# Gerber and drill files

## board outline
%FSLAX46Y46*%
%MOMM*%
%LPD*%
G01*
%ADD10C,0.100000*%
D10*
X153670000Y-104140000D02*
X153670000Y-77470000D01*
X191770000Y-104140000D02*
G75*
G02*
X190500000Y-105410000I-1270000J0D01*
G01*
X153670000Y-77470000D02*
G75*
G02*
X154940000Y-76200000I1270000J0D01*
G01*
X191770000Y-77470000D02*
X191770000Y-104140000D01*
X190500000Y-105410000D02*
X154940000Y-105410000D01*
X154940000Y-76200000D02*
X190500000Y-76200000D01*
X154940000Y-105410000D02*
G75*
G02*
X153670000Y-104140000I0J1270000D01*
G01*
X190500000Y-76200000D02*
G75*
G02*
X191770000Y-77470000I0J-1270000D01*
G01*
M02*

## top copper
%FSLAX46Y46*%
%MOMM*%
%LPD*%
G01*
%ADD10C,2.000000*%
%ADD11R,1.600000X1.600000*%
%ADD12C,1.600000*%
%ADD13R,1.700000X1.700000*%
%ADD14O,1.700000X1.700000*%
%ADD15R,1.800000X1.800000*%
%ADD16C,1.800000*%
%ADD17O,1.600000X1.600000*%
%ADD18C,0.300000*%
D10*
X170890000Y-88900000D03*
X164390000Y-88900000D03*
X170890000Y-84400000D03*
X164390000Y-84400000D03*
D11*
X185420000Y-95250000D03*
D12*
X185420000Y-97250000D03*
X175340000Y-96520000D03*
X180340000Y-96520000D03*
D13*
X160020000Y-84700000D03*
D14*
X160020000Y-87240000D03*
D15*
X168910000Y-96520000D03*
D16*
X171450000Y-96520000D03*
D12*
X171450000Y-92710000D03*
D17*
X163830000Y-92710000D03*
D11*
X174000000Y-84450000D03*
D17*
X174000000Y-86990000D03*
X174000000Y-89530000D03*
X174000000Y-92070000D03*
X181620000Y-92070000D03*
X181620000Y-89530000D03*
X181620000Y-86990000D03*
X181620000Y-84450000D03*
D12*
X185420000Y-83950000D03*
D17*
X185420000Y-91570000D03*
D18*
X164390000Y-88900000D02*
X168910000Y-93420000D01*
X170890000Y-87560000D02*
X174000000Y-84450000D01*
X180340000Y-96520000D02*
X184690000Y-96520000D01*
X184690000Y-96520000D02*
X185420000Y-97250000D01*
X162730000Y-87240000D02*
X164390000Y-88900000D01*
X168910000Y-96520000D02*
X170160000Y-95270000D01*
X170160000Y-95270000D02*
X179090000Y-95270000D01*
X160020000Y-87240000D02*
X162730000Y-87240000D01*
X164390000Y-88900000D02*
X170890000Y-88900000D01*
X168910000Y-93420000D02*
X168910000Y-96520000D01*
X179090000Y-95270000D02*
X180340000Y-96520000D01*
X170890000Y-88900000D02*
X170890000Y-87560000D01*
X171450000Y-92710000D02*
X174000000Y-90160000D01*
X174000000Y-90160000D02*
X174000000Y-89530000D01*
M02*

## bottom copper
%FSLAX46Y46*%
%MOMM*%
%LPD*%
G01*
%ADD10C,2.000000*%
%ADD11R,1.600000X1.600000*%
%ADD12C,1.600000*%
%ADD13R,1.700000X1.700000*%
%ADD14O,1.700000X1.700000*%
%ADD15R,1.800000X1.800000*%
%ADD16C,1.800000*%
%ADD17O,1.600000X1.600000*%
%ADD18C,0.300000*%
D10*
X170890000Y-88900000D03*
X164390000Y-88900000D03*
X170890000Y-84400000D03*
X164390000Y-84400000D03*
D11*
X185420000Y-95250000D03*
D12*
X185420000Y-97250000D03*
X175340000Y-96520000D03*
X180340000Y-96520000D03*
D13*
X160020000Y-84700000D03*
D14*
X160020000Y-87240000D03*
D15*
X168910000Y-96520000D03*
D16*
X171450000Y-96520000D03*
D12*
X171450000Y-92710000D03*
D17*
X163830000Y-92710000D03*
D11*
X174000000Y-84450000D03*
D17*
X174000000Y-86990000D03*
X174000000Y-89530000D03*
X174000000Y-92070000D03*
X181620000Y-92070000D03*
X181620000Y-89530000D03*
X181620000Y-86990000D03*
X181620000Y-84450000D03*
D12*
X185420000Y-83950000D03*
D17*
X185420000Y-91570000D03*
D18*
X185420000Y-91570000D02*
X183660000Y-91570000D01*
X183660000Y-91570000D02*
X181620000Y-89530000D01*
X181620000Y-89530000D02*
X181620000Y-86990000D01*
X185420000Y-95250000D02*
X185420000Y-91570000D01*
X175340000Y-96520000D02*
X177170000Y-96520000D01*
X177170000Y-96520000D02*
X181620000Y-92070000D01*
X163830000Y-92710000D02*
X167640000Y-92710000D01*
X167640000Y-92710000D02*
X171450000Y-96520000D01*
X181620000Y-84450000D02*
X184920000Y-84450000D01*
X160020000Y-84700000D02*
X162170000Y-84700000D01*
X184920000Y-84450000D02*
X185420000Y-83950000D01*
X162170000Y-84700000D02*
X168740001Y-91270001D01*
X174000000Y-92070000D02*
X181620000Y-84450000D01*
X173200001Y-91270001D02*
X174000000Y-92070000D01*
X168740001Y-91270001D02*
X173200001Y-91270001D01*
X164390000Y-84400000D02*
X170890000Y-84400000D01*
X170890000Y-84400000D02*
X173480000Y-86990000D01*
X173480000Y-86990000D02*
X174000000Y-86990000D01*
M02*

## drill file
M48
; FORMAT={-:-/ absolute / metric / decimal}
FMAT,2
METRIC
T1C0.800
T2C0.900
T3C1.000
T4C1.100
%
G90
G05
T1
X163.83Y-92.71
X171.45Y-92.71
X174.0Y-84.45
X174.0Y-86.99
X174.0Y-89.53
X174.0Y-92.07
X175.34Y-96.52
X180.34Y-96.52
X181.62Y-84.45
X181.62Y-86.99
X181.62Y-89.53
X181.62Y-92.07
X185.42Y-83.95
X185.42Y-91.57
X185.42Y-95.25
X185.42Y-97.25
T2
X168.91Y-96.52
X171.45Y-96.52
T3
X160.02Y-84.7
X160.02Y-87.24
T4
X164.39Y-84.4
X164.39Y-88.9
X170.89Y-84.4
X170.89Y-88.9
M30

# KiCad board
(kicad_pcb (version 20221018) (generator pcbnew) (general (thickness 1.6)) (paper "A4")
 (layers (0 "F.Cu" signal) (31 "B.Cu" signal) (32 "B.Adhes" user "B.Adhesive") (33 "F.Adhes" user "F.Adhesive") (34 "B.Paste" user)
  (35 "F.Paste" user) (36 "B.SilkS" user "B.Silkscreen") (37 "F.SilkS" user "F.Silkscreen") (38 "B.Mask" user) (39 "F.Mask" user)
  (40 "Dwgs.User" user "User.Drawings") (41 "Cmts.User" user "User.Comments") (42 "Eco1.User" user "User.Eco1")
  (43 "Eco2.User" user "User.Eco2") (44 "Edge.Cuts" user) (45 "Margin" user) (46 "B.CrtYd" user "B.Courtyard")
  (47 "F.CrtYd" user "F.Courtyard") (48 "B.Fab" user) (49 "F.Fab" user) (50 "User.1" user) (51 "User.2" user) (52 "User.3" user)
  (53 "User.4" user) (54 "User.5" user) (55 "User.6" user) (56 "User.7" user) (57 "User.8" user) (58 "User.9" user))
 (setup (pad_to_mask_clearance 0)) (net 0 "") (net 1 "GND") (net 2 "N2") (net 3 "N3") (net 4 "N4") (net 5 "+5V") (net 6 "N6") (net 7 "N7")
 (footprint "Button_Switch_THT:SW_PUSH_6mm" (layer "F.Cu") (at 170.89 88.9 180)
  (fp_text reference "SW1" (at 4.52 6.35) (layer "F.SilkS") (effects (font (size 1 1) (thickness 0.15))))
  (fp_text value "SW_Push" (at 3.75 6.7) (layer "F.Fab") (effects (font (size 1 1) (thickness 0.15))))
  (pad "1" thru_hole circle (at 0 0 270) (size 2 2) (drill 1.1) (layers "*.Cu" "*.Mask") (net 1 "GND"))
  (pad "1" thru_hole circle (at 6.5 0 270) (size 2 2) (drill 1.1) (layers "*.Cu" "*.Mask") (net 1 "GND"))
  (pad "2" thru_hole circle (at 0 4.5 270) (size 2 2) (drill 1.1) (layers "*.Cu" "*.Mask") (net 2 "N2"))
  (pad "2" thru_hole circle (at 6.5 4.5 270) (size 2 2) (drill 1.1) (layers "*.Cu" "*.Mask") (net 2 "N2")))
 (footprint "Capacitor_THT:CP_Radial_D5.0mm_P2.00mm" (layer "F.Cu") (at 185.42 95.25 -90)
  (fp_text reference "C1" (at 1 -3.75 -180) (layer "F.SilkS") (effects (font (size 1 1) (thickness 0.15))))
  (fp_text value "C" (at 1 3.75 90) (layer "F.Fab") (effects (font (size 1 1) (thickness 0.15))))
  (pad "1" thru_hole rect (at 0 0 270) (size 1.6 1.6) (drill 0.8) (layers "*.Cu" "*.Mask") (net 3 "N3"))
  (pad "2" thru_hole circle (at 2 0 270) (size 1.6 1.6) (drill 0.8) (layers "*.Cu" "*.Mask") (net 1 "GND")))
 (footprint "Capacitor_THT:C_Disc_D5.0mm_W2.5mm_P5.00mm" (layer "F.Cu") (at 175.34 96.52)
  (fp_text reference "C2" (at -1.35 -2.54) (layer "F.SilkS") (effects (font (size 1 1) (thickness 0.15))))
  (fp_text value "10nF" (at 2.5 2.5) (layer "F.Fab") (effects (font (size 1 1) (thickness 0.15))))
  (pad "1" thru_hole circle (at 0 0) (size 1.6 1.6) (drill 0.8) (layers "*.Cu" "*.Mask") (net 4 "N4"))
  (pad "2" thru_hole circle (at 5 0) (size 1.6 1.6) (drill 0.8) (layers "*.Cu" "*.Mask") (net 1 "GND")))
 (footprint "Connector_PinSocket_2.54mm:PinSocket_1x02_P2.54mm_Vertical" (layer "F.Cu") (at 160.02 84.7)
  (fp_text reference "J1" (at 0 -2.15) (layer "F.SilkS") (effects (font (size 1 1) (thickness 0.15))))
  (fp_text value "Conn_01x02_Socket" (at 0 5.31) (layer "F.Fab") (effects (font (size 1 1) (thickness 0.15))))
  (pad "1" thru_hole rect (at 0 0) (size 1.7 1.7) (drill 1) (layers "*.Cu" "*.Mask") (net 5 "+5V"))
  (pad "2" thru_hole oval (at 0 2.54) (size 1.7 1.7) (drill 1) (layers "*.Cu" "*.Mask") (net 1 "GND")))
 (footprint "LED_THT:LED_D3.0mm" (layer "F.Cu") (at 168.91 96.52)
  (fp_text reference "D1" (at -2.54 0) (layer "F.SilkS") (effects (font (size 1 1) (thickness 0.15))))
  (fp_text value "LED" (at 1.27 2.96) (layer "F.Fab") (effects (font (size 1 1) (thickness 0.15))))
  (pad "1" thru_hole rect (at 0 0) (size 1.8 1.8) (drill 0.9) (layers "*.Cu" "*.Mask") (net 1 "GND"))
  (pad "2" thru_hole circle (at 2.54 0) (size 1.8 1.8) (drill 0.9) (layers "*.Cu" "*.Mask") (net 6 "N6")))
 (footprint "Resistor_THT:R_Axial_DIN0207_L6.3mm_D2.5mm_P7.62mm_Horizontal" (layer "F.Cu") (at 171.45 92.71 180)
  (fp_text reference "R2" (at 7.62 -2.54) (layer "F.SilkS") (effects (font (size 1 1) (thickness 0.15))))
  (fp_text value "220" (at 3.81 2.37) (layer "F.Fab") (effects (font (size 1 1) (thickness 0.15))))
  (pad "1" thru_hole circle (at 0 0 180) (size 1.6 1.6) (drill 0.8) (layers "*.Cu" "*.Mask") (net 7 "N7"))
  (pad "2" thru_hole oval (at 7.62 0 180) (size 1.6 1.6) (drill 0.8) (layers "*.Cu" "*.Mask") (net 6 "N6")))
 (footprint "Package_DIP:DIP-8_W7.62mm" (layer "F.Cu") (at 174 84.45)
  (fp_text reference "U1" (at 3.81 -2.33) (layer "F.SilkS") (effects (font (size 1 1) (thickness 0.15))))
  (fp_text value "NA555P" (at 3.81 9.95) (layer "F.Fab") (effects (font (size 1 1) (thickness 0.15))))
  (pad "1" thru_hole rect (at 0 0) (size 1.6 1.6) (drill 0.8) (layers "*.Cu" "*.Mask") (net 1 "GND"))
  (pad "2" thru_hole oval (at 0 2.54) (size 1.6 1.6) (drill 0.8) (layers "*.Cu" "*.Mask") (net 2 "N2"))
  (pad "3" thru_hole oval (at 0 5.08) (size 1.6 1.6) (drill 0.8) (layers "*.Cu" "*.Mask") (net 7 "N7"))
  (pad "4" thru_hole oval (at 0 7.62) (size 1.6 1.6) (drill 0.8) (layers "*.Cu" "*.Mask") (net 5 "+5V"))
  (pad "5" thru_hole oval (at 7.62 7.62) (size 1.6 1.6) (drill 0.8) (layers "*.Cu" "*.Mask") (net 4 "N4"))
  (pad "6" thru_hole oval (at 7.62 5.08) (size 1.6 1.6) (drill 0.8) (layers "*.Cu" "*.Mask") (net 3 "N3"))
  (pad "7" thru_hole oval (at 7.62 2.54) (size 1.6 1.6) (drill 0.8) (layers "*.Cu" "*.Mask") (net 3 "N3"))
  (pad "8" thru_hole oval (at 7.62 0) (size 1.6 1.6) (drill 0.8) (layers "*.Cu" "*.Mask") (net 5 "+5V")))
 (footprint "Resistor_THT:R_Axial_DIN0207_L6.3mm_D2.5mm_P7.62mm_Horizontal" (layer "F.Cu") (at 185.42 83.95 -90)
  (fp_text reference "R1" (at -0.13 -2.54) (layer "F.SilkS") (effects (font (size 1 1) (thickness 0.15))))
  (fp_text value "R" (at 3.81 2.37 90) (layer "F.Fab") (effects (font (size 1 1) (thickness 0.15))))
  (pad "1" thru_hole circle (at 0 0 270) (size 1.6 1.6) (drill 0.8) (layers "*.Cu" "*.Mask") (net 5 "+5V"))
  (pad "2" thru_hole oval (at 7.62 0 270) (size 1.6 1.6) (drill 0.8) (layers "*.Cu" "*.Mask") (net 3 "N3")))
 (gr_line (start 153.67 104.14) (end 153.67 77.47) (stroke (width 0.1) (type default)) (layer "Edge.Cuts"))
 (gr_arc (start 191.77 104.14) (mid 191.398026 105.038026) (end 190.5 105.41) (stroke (width 0.1) (type default)) (layer "Edge.Cuts"))
 (gr_arc (start 153.67 77.47) (mid 154.041974 76.571974) (end 154.94 76.2) (stroke (width 0.1) (type default)) (layer "Edge.Cuts"))
 (gr_line (start 191.77 77.47) (end 191.77 104.14) (stroke (width 0.1) (type default)) (layer "Edge.Cuts"))
 (gr_line (start 190.5 105.41) (end 154.94 105.41) (stroke (width 0.1) (type default)) (layer "Edge.Cuts"))
 (gr_line (start 154.94 76.2) (end 190.5 76.2) (stroke (width 0.1) (type default)) (layer "Edge.Cuts"))
 (gr_arc (start 154.94 105.41) (mid 154.041974 105.038026) (end 153.67 104.14) (stroke (width 0.1) (type default)) (layer "Edge.Cuts"))
 (gr_arc (start 190.5 76.2) (mid 191.398026 76.571974) (end 191.77 77.47) (stroke (width 0.1) (type default)) (layer "Edge.Cuts"))
 (segment (start 185.42 91.57) (end 183.66 91.57) (width 0.3) (layer "B.Cu") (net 3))
 (segment (start 183.66 91.57) (end 181.62 89.53) (width 0.3) (layer "B.Cu") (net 3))
 (segment (start 181.62 89.53) (end 181.62 86.99) (width 0.3) (layer "B.Cu") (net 3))
 (segment (start 185.42 95.25) (end 185.42 91.57) (width 0.3) (layer "B.Cu") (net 3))
 (segment (start 164.39 88.9) (end 168.91 93.42) (width 0.3) (layer "F.Cu") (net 1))
 (segment (start 170.89 87.56) (end 174 84.45) (width 0.3) (layer "F.Cu") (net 1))
 (segment (start 180.34 96.52) (end 184.69 96.52) (width 0.3) (layer "F.Cu") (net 1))
 (segment (start 184.69 96.52) (end 185.42 97.25) (width 0.3) (layer "F.Cu") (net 1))
 (segment (start 162.73 87.24) (end 164.39 88.9) (width 0.3) (layer "F.Cu") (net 1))
 (segment (start 168.91 96.52) (end 170.16 95.27) (width 0.3) (layer "F.Cu") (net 1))
 (segment (start 170.16 95.27) (end 179.09 95.27) (width 0.3) (layer "F.Cu") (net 1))
 (segment (start 160.02 87.24) (end 162.73 87.24) (width 0.3) (layer "F.Cu") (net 1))
 (segment (start 164.39 88.9) (end 170.89 88.9) (width 0.3) (layer "F.Cu") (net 1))
 (segment (start 168.91 93.42) (end 168.91 96.52) (width 0.3) (layer "F.Cu") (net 1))
 (segment (start 179.09 95.27) (end 180.34 96.52) (width 0.3) (layer "F.Cu") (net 1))
 (segment (start 170.89 88.9) (end 170.89 87.56) (width 0.3) (layer "F.Cu") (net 1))
 (segment (start 175.34 96.52) (end 177.17 96.52) (width 0.3) (layer "B.Cu") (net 4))
 (segment (start 177.17 96.52) (end 181.62 92.07) (width 0.3) (layer "B.Cu") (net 4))
 (segment (start 163.83 92.71) (end 167.64 92.71) (width 0.3) (layer "B.Cu") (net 6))
 (segment (start 167.64 92.71) (end 171.45 96.52) (width 0.3) (layer "B.Cu") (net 6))
 (segment (start 181.62 84.45) (end 184.92 84.45) (width 0.3) (layer "B.Cu") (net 5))
 (segment (start 160.02 84.7) (end 162.17 84.7) (width 0.3) (layer "B.Cu") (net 5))
 (segment (start 184.92 84.45) (end 185.42 83.95) (width 0.3) (layer "B.Cu") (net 5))
 (segment (start 162.17 84.7) (end 168.740001 91.270001) (width 0.3) (layer "B.Cu") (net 5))
 (segment (start 174 92.07) (end 181.62 84.45) (width 0.3) (layer "B.Cu") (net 5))
 (segment (start 173.200001 91.270001) (end 174 92.07) (width 0.3) (layer "B.Cu") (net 5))
 (segment (start 168.740001 91.270001) (end 173.200001 91.270001) (width 0.3) (layer "B.Cu") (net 5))
 (segment (start 171.45 92.71) (end 174 90.16) (width 0.3) (layer "F.Cu") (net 7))
 (segment (start 174 90.16) (end 174 89.53) (width 0.3) (layer "F.Cu") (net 7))
 (segment (start 164.39 84.4) (end 170.89 84.4) (width 0.3) (layer "B.Cu") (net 2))
 (segment (start 170.89 84.4) (end 173.48 86.99) (width 0.3) (layer "B.Cu") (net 2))
 (segment (start 173.48 86.99) (end 174 86.99) (width 0.3) (layer "B.Cu") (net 2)))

